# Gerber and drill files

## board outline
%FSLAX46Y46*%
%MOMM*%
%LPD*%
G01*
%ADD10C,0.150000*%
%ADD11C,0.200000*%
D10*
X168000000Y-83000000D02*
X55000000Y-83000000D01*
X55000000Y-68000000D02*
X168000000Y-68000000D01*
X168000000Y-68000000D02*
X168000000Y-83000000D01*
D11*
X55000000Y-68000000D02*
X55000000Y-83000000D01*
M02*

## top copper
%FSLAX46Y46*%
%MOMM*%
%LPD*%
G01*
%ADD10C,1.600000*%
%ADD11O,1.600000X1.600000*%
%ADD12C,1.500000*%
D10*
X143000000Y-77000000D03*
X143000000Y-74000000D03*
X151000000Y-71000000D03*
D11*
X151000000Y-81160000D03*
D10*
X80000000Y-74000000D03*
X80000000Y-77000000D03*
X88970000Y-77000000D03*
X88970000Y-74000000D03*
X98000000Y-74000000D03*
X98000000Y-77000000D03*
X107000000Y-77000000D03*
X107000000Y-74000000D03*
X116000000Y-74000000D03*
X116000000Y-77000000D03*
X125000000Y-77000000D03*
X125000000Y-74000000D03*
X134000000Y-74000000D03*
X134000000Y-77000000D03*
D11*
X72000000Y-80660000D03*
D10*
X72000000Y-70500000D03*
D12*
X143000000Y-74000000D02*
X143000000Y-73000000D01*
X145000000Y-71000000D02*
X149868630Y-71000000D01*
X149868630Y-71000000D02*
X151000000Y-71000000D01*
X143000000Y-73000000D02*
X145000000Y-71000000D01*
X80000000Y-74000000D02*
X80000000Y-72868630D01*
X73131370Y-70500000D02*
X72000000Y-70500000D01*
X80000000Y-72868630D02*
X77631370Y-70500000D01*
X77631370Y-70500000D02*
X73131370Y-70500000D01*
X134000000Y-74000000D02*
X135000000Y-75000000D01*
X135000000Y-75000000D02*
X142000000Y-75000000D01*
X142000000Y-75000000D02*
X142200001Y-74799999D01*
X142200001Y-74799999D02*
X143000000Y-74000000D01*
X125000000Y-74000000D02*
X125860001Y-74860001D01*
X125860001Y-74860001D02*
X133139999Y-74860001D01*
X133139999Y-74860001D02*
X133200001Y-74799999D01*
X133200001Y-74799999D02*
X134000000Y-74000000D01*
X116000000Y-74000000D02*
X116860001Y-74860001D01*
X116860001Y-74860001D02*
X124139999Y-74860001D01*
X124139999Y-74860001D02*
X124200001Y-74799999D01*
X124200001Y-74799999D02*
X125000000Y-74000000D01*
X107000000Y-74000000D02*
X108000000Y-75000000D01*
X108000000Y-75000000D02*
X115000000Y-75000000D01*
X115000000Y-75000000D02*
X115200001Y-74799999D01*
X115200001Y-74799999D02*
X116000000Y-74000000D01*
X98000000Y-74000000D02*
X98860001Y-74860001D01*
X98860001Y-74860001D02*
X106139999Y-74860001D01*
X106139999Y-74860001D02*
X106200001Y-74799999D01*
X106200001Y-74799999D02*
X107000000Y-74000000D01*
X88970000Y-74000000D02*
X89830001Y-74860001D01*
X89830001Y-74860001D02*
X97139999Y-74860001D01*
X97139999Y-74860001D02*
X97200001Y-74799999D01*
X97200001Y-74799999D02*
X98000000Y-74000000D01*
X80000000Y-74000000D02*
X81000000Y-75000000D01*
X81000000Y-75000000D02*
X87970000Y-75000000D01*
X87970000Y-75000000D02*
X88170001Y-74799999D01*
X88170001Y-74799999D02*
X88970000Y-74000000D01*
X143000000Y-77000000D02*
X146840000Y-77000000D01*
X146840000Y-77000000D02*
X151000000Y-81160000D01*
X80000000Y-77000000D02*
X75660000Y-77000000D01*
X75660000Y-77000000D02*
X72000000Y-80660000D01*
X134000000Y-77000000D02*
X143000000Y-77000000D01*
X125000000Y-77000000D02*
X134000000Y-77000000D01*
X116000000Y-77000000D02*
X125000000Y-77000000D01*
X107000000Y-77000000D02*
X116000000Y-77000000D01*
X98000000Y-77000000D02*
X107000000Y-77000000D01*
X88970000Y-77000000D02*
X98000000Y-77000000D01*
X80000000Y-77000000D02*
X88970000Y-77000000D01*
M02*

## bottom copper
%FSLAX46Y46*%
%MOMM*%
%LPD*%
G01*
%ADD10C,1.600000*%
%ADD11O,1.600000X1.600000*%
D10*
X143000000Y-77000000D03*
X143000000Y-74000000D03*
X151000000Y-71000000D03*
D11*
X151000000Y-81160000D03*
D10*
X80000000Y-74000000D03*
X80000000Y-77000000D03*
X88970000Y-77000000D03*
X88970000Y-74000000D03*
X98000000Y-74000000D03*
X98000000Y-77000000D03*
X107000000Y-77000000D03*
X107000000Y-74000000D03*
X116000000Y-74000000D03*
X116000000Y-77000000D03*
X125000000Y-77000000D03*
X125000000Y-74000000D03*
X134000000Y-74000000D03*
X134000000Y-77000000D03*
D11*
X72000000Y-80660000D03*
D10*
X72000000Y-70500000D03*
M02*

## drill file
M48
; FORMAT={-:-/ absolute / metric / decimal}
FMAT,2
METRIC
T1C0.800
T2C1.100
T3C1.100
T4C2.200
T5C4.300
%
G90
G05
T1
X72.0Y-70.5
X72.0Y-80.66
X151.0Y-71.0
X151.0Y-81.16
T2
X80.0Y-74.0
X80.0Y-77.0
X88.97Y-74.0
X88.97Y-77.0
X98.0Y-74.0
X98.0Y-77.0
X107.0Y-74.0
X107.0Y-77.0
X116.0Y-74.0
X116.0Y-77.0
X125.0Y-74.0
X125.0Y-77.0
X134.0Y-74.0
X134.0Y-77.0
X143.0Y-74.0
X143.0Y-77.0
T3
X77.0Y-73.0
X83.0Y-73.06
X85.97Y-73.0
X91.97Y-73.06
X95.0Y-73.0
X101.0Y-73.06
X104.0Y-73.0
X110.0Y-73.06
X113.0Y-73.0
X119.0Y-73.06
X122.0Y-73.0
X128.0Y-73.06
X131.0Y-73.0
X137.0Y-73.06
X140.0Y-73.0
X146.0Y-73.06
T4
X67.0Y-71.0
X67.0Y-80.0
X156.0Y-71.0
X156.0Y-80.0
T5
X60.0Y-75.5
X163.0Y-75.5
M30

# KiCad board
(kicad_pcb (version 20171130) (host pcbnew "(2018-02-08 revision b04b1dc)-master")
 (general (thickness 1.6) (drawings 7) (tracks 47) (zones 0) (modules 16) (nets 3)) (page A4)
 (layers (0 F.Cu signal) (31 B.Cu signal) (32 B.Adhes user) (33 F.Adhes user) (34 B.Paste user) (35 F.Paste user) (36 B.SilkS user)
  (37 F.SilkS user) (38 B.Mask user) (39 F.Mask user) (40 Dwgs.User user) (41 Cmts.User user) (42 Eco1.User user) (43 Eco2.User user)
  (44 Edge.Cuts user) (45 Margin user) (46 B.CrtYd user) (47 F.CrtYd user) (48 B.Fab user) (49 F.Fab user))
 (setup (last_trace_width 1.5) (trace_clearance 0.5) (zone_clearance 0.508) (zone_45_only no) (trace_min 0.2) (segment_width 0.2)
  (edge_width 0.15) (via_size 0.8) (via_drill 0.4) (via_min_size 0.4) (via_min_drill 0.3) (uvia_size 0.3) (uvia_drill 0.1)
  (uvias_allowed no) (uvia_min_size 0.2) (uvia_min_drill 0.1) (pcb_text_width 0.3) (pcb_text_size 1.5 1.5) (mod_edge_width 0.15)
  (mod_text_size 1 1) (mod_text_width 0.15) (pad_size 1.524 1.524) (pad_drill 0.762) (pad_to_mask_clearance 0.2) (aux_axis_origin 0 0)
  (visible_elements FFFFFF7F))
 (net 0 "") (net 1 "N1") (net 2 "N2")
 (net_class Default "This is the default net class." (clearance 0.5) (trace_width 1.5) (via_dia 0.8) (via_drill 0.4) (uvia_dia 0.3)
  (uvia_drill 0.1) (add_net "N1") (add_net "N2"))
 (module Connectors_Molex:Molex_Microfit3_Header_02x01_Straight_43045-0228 (layer F.Cu) (at 143 77)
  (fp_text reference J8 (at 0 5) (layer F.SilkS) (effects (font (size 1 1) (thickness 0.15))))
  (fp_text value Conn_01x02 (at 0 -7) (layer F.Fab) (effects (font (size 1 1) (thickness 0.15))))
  (pad "" np_thru_hole circle (at -3 -4) (size 1.1 1.1) (drill 1.1) (layers *.Cu *.Mask))
  (pad 1 thru_hole circle (at 0 0) (size 1.6 1.6) (drill 1.1) (layers *.Cu *.Mask) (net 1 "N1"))
  (pad 2 thru_hole circle (at 0 -3) (size 1.6 1.6) (drill 1.1) (layers *.Cu *.Mask) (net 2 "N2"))
  (pad "" np_thru_hole circle (at 3 -3.94) (size 1.1 1.1) (drill 1.1) (layers *.Cu *.Mask)))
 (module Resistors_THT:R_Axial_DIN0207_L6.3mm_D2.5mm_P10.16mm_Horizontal (layer F.Cu) (at 151 71 270)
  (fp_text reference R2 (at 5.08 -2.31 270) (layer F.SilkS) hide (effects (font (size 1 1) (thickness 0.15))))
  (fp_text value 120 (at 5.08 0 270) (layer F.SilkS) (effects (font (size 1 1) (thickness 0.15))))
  (pad 1 thru_hole circle (at 0 0 270) (size 1.6 1.6) (drill 0.8) (layers *.Cu *.Mask) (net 2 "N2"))
  (pad 2 thru_hole oval (at 10.16 0 270) (size 1.6 1.6) (drill 0.8) (layers *.Cu *.Mask) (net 1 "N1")))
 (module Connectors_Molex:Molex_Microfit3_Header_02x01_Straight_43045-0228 (layer F.Cu) (at 80 77)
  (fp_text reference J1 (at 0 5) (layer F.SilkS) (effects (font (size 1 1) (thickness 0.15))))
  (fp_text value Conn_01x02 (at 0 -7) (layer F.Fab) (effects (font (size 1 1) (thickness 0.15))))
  (pad "" np_thru_hole circle (at 3 -3.94) (size 1.1 1.1) (drill 1.1) (layers *.Cu *.Mask))
  (pad 2 thru_hole circle (at 0 -3) (size 1.6 1.6) (drill 1.1) (layers *.Cu *.Mask) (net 2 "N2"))
  (pad 1 thru_hole circle (at 0 0) (size 1.6 1.6) (drill 1.1) (layers *.Cu *.Mask) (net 1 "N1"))
  (pad "" np_thru_hole circle (at -3 -4) (size 1.1 1.1) (drill 1.1) (layers *.Cu *.Mask)))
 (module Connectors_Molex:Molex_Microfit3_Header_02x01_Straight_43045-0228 (layer F.Cu) (at 88.97 77)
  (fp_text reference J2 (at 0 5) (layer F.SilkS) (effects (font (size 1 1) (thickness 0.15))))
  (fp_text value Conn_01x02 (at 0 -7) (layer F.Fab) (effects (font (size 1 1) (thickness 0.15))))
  (pad "" np_thru_hole circle (at -3 -4) (size 1.1 1.1) (drill 1.1) (layers *.Cu *.Mask))
  (pad 1 thru_hole circle (at 0 0) (size 1.6 1.6) (drill 1.1) (layers *.Cu *.Mask) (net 1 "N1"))
  (pad 2 thru_hole circle (at 0 -3) (size 1.6 1.6) (drill 1.1) (layers *.Cu *.Mask) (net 2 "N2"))
  (pad "" np_thru_hole circle (at 3 -3.94) (size 1.1 1.1) (drill 1.1) (layers *.Cu *.Mask)))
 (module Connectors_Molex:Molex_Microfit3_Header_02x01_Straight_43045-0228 (layer F.Cu) (at 98 77)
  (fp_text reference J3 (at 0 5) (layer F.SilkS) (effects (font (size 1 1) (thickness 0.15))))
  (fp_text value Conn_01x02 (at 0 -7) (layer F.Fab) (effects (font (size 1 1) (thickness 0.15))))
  (pad "" np_thru_hole circle (at 3 -3.94) (size 1.1 1.1) (drill 1.1) (layers *.Cu *.Mask))
  (pad 2 thru_hole circle (at 0 -3) (size 1.6 1.6) (drill 1.1) (layers *.Cu *.Mask) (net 2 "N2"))
  (pad 1 thru_hole circle (at 0 0) (size 1.6 1.6) (drill 1.1) (layers *.Cu *.Mask) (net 1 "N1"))
  (pad "" np_thru_hole circle (at -3 -4) (size 1.1 1.1) (drill 1.1) (layers *.Cu *.Mask)))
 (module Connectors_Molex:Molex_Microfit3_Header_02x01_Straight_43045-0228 (layer F.Cu) (at 107 77)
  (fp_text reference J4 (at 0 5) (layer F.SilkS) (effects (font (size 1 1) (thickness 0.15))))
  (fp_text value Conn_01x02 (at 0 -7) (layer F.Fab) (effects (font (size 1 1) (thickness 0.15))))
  (pad "" np_thru_hole circle (at -3 -4) (size 1.1 1.1) (drill 1.1) (layers *.Cu *.Mask))
  (pad 1 thru_hole circle (at 0 0) (size 1.6 1.6) (drill 1.1) (layers *.Cu *.Mask) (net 1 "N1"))
  (pad 2 thru_hole circle (at 0 -3) (size 1.6 1.6) (drill 1.1) (layers *.Cu *.Mask) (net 2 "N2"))
  (pad "" np_thru_hole circle (at 3 -3.94) (size 1.1 1.1) (drill 1.1) (layers *.Cu *.Mask)))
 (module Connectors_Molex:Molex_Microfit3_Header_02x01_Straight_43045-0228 (layer F.Cu) (at 116 77)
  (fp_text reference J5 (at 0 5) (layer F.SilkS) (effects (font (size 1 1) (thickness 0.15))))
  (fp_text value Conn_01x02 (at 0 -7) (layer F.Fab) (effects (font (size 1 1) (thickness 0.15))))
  (pad "" np_thru_hole circle (at 3 -3.94) (size 1.1 1.1) (drill 1.1) (layers *.Cu *.Mask))
  (pad 2 thru_hole circle (at 0 -3) (size 1.6 1.6) (drill 1.1) (layers *.Cu *.Mask) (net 2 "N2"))
  (pad 1 thru_hole circle (at 0 0) (size 1.6 1.6) (drill 1.1) (layers *.Cu *.Mask) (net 1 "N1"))
  (pad "" np_thru_hole circle (at -3 -4) (size 1.1 1.1) (drill 1.1) (layers *.Cu *.Mask)))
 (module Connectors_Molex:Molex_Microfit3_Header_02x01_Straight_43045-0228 (layer F.Cu) (at 125 77)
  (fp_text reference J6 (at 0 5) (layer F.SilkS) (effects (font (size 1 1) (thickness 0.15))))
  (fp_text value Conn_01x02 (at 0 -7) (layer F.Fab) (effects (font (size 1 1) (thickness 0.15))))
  (pad "" np_thru_hole circle (at -3 -4) (size 1.1 1.1) (drill 1.1) (layers *.Cu *.Mask))
  (pad 1 thru_hole circle (at 0 0) (size 1.6 1.6) (drill 1.1) (layers *.Cu *.Mask) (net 1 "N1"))
  (pad 2 thru_hole circle (at 0 -3) (size 1.6 1.6) (drill 1.1) (layers *.Cu *.Mask) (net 2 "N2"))
  (pad "" np_thru_hole circle (at 3 -3.94) (size 1.1 1.1) (drill 1.1) (layers *.Cu *.Mask)))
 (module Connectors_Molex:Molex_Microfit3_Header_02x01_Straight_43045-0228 (layer F.Cu) (at 134 77)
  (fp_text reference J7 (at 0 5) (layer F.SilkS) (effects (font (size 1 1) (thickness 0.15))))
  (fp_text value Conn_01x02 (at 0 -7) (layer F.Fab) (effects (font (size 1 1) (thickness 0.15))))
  (pad "" np_thru_hole circle (at 3 -3.94) (size 1.1 1.1) (drill 1.1) (layers *.Cu *.Mask))
  (pad 2 thru_hole circle (at 0 -3) (size 1.6 1.6) (drill 1.1) (layers *.Cu *.Mask) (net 2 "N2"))
  (pad 1 thru_hole circle (at 0 0) (size 1.6 1.6) (drill 1.1) (layers *.Cu *.Mask) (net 1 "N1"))
  (pad "" np_thru_hole circle (at -3 -4) (size 1.1 1.1) (drill 1.1) (layers *.Cu *.Mask)))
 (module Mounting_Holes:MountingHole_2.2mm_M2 (layer F.Cu) (at 67 71)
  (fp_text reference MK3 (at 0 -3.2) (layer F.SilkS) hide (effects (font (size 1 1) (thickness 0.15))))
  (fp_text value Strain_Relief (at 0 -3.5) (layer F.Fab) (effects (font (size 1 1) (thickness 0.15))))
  (pad 1 np_thru_hole circle (at 0 0) (size 2.2 2.2) (drill 2.2) (layers *.Cu *.Mask)))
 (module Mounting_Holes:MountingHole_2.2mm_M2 (layer F.Cu) (at 67 80)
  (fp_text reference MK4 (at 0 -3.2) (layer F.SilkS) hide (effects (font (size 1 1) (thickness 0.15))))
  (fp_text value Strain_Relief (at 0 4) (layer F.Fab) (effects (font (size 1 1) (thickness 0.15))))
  (pad 1 np_thru_hole circle (at 0 0) (size 2.2 2.2) (drill 2.2) (layers *.Cu *.Mask)))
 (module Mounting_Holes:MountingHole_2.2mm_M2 (layer F.Cu) (at 156 71)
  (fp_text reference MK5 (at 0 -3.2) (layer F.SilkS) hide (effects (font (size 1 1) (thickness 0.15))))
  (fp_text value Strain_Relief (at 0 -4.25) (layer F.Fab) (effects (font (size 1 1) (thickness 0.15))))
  (pad 1 np_thru_hole circle (at 0 0) (size 2.2 2.2) (drill 2.2) (layers *.Cu *.Mask)))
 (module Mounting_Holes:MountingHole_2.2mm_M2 (layer F.Cu) (at 156 80)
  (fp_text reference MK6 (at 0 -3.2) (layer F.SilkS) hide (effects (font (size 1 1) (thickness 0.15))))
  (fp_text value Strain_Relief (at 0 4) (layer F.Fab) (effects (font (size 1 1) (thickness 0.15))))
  (pad 1 np_thru_hole circle (at 0 0) (size 2.2 2.2) (drill 2.2) (layers *.Cu *.Mask)))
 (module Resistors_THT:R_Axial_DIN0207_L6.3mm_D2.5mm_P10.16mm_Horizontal (layer F.Cu) (at 72 70.5 270)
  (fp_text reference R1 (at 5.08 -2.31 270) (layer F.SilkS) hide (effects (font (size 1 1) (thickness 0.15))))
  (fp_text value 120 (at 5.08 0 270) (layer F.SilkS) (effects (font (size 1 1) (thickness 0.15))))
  (pad 2 thru_hole oval (at 10.16 0 270) (size 1.6 1.6) (drill 0.8) (layers *.Cu *.Mask) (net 1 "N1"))
  (pad 1 thru_hole circle (at 0 0 270) (size 1.6 1.6) (drill 0.8) (layers *.Cu *.Mask) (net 2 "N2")))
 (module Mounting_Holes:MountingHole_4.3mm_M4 (layer F.Cu) (at 60 75.5)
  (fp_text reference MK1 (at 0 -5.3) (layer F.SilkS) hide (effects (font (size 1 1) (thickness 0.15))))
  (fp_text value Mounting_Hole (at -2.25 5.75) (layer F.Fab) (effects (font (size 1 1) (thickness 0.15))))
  (pad 1 np_thru_hole circle (at 0 0) (size 4.3 4.3) (drill 4.3) (layers *.Cu *.Mask)))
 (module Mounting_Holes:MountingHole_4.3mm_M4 (layer F.Cu) (at 163 75.5)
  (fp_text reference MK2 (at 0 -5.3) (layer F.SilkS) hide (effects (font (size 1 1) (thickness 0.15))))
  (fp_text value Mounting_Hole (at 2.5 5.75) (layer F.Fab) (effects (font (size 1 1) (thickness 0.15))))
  (pad 1 np_thru_hole circle (at 0 0) (size 4.3 4.3) (drill 4.3) (layers *.Cu *.Mask)))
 (gr_line (start 168 83) (end 55 83) (layer Edge.Cuts) (width 0.15))
 (gr_line (start 55 68) (end 168 68) (layer Edge.Cuts) (width 0.15))
 (gr_line (start 168 68) (end 168 83) (layer Edge.Cuts) (width 0.15))
 (gr_line (start 55 68) (end 55 83) (layer Edge.Cuts) (width 0.2))
 (segment (start 143 74) (end 143 73) (width 1.5) (layer F.Cu) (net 2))
 (segment (start 145 71) (end 149.86863 71) (width 1.5) (layer F.Cu) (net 2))
 (segment (start 149.86863 71) (end 151 71) (width 1.5) (layer F.Cu) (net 2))
 (segment (start 143 73) (end 145 71) (width 1.5) (layer F.Cu) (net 2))
 (segment (start 80 74) (end 80 72.86863) (width 1.5) (layer F.Cu) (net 2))
 (segment (start 73.13137 70.5) (end 72 70.5) (width 1.5) (layer F.Cu) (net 2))
 (segment (start 80 72.86863) (end 77.63137 70.5) (width 1.5) (layer F.Cu) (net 2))
 (segment (start 77.63137 70.5) (end 73.13137 70.5) (width 1.5) (layer F.Cu) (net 2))
 (segment (start 134 74) (end 135 75) (width 1.5) (layer F.Cu) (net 2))
 (segment (start 135 75) (end 142 75) (width 1.5) (layer F.Cu) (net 2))
 (segment (start 142 75) (end 142.200001 74.799999) (width 1.5) (layer F.Cu) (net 2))
 (segment (start 142.200001 74.799999) (end 143 74) (width 1.5) (layer F.Cu) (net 2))
 (segment (start 125 74) (end 125.860001 74.860001) (width 1.5) (layer F.Cu) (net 2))
 (segment (start 125.860001 74.860001) (end 133.139999 74.860001) (width 1.5) (layer F.Cu) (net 2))
 (segment (start 133.139999 74.860001) (end 133.200001 74.799999) (width 1.5) (layer F.Cu) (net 2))
 (segment (start 133.200001 74.799999) (end 134 74) (width 1.5) (layer F.Cu) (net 2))
 (segment (start 116 74) (end 116.860001 74.860001) (width 1.5) (layer F.Cu) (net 2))
 (segment (start 116.860001 74.860001) (end 124.139999 74.860001) (width 1.5) (layer F.Cu) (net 2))
 (segment (start 124.139999 74.860001) (end 124.200001 74.799999) (width 1.5) (layer F.Cu) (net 2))
 (segment (start 124.200001 74.799999) (end 125 74) (width 1.5) (layer F.Cu) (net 2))
 (segment (start 107 74) (end 108 75) (width 1.5) (layer F.Cu) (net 2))
 (segment (start 108 75) (end 115 75) (width 1.5) (layer F.Cu) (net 2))
 (segment (start 115 75) (end 115.200001 74.799999) (width 1.5) (layer F.Cu) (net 2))
 (segment (start 115.200001 74.799999) (end 116 74) (width 1.5) (layer F.Cu) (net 2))
 (segment (start 98 74) (end 98.860001 74.860001) (width 1.5) (layer F.Cu) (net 2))
 (segment (start 98.860001 74.860001) (end 106.139999 74.860001) (width 1.5) (layer F.Cu) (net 2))
 (segment (start 106.139999 74.860001) (end 106.200001 74.799999) (width 1.5) (layer F.Cu) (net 2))
 (segment (start 106.200001 74.799999) (end 107 74) (width 1.5) (layer F.Cu) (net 2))
 (segment (start 88.97 74) (end 89.830001 74.860001) (width 1.5) (layer F.Cu) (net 2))
 (segment (start 89.830001 74.860001) (end 97.139999 74.860001) (width 1.5) (layer F.Cu) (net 2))
 (segment (start 97.139999 74.860001) (end 97.200001 74.799999) (width 1.5) (layer F.Cu) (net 2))
 (segment (start 97.200001 74.799999) (end 98 74) (width 1.5) (layer F.Cu) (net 2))
 (segment (start 80 74) (end 81 75) (width 1.5) (layer F.Cu) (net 2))
 (segment (start 81 75) (end 87.97 75) (width 1.5) (layer F.Cu) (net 2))
 (segment (start 87.97 75) (end 88.170001 74.799999) (width 1.5) (layer F.Cu) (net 2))
 (segment (start 88.170001 74.799999) (end 88.97 74) (width 1.5) (layer F.Cu) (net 2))
 (segment (start 143 77) (end 146.84 77) (width 1.5) (layer F.Cu) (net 1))
 (segment (start 146.84 77) (end 151 81.16) (width 1.5) (layer F.Cu) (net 1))
 (segment (start 80 77) (end 75.66 77) (width 1.5) (layer F.Cu) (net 1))
 (segment (start 75.66 77) (end 72 80.66) (width 1.5) (layer F.Cu) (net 1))
 (segment (start 134 77) (end 143 77) (width 1.5) (layer F.Cu) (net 1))
 (segment (start 125 77) (end 134 77) (width 1.5) (layer F.Cu) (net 1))
 (segment (start 116 77) (end 125 77) (width 1.5) (layer F.Cu) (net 1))
 (segment (start 107 77) (end 116 77) (width 1.5) (layer F.Cu) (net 1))
 (segment (start 98 77) (end 107 77) (width 1.5) (layer F.Cu) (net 1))
 (segment (start 88.97 77) (end 98 77) (width 1.5) (layer F.Cu) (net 1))
 (segment (start 80 77) (end 88.97 77) (width 1.5) (layer F.Cu) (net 1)))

